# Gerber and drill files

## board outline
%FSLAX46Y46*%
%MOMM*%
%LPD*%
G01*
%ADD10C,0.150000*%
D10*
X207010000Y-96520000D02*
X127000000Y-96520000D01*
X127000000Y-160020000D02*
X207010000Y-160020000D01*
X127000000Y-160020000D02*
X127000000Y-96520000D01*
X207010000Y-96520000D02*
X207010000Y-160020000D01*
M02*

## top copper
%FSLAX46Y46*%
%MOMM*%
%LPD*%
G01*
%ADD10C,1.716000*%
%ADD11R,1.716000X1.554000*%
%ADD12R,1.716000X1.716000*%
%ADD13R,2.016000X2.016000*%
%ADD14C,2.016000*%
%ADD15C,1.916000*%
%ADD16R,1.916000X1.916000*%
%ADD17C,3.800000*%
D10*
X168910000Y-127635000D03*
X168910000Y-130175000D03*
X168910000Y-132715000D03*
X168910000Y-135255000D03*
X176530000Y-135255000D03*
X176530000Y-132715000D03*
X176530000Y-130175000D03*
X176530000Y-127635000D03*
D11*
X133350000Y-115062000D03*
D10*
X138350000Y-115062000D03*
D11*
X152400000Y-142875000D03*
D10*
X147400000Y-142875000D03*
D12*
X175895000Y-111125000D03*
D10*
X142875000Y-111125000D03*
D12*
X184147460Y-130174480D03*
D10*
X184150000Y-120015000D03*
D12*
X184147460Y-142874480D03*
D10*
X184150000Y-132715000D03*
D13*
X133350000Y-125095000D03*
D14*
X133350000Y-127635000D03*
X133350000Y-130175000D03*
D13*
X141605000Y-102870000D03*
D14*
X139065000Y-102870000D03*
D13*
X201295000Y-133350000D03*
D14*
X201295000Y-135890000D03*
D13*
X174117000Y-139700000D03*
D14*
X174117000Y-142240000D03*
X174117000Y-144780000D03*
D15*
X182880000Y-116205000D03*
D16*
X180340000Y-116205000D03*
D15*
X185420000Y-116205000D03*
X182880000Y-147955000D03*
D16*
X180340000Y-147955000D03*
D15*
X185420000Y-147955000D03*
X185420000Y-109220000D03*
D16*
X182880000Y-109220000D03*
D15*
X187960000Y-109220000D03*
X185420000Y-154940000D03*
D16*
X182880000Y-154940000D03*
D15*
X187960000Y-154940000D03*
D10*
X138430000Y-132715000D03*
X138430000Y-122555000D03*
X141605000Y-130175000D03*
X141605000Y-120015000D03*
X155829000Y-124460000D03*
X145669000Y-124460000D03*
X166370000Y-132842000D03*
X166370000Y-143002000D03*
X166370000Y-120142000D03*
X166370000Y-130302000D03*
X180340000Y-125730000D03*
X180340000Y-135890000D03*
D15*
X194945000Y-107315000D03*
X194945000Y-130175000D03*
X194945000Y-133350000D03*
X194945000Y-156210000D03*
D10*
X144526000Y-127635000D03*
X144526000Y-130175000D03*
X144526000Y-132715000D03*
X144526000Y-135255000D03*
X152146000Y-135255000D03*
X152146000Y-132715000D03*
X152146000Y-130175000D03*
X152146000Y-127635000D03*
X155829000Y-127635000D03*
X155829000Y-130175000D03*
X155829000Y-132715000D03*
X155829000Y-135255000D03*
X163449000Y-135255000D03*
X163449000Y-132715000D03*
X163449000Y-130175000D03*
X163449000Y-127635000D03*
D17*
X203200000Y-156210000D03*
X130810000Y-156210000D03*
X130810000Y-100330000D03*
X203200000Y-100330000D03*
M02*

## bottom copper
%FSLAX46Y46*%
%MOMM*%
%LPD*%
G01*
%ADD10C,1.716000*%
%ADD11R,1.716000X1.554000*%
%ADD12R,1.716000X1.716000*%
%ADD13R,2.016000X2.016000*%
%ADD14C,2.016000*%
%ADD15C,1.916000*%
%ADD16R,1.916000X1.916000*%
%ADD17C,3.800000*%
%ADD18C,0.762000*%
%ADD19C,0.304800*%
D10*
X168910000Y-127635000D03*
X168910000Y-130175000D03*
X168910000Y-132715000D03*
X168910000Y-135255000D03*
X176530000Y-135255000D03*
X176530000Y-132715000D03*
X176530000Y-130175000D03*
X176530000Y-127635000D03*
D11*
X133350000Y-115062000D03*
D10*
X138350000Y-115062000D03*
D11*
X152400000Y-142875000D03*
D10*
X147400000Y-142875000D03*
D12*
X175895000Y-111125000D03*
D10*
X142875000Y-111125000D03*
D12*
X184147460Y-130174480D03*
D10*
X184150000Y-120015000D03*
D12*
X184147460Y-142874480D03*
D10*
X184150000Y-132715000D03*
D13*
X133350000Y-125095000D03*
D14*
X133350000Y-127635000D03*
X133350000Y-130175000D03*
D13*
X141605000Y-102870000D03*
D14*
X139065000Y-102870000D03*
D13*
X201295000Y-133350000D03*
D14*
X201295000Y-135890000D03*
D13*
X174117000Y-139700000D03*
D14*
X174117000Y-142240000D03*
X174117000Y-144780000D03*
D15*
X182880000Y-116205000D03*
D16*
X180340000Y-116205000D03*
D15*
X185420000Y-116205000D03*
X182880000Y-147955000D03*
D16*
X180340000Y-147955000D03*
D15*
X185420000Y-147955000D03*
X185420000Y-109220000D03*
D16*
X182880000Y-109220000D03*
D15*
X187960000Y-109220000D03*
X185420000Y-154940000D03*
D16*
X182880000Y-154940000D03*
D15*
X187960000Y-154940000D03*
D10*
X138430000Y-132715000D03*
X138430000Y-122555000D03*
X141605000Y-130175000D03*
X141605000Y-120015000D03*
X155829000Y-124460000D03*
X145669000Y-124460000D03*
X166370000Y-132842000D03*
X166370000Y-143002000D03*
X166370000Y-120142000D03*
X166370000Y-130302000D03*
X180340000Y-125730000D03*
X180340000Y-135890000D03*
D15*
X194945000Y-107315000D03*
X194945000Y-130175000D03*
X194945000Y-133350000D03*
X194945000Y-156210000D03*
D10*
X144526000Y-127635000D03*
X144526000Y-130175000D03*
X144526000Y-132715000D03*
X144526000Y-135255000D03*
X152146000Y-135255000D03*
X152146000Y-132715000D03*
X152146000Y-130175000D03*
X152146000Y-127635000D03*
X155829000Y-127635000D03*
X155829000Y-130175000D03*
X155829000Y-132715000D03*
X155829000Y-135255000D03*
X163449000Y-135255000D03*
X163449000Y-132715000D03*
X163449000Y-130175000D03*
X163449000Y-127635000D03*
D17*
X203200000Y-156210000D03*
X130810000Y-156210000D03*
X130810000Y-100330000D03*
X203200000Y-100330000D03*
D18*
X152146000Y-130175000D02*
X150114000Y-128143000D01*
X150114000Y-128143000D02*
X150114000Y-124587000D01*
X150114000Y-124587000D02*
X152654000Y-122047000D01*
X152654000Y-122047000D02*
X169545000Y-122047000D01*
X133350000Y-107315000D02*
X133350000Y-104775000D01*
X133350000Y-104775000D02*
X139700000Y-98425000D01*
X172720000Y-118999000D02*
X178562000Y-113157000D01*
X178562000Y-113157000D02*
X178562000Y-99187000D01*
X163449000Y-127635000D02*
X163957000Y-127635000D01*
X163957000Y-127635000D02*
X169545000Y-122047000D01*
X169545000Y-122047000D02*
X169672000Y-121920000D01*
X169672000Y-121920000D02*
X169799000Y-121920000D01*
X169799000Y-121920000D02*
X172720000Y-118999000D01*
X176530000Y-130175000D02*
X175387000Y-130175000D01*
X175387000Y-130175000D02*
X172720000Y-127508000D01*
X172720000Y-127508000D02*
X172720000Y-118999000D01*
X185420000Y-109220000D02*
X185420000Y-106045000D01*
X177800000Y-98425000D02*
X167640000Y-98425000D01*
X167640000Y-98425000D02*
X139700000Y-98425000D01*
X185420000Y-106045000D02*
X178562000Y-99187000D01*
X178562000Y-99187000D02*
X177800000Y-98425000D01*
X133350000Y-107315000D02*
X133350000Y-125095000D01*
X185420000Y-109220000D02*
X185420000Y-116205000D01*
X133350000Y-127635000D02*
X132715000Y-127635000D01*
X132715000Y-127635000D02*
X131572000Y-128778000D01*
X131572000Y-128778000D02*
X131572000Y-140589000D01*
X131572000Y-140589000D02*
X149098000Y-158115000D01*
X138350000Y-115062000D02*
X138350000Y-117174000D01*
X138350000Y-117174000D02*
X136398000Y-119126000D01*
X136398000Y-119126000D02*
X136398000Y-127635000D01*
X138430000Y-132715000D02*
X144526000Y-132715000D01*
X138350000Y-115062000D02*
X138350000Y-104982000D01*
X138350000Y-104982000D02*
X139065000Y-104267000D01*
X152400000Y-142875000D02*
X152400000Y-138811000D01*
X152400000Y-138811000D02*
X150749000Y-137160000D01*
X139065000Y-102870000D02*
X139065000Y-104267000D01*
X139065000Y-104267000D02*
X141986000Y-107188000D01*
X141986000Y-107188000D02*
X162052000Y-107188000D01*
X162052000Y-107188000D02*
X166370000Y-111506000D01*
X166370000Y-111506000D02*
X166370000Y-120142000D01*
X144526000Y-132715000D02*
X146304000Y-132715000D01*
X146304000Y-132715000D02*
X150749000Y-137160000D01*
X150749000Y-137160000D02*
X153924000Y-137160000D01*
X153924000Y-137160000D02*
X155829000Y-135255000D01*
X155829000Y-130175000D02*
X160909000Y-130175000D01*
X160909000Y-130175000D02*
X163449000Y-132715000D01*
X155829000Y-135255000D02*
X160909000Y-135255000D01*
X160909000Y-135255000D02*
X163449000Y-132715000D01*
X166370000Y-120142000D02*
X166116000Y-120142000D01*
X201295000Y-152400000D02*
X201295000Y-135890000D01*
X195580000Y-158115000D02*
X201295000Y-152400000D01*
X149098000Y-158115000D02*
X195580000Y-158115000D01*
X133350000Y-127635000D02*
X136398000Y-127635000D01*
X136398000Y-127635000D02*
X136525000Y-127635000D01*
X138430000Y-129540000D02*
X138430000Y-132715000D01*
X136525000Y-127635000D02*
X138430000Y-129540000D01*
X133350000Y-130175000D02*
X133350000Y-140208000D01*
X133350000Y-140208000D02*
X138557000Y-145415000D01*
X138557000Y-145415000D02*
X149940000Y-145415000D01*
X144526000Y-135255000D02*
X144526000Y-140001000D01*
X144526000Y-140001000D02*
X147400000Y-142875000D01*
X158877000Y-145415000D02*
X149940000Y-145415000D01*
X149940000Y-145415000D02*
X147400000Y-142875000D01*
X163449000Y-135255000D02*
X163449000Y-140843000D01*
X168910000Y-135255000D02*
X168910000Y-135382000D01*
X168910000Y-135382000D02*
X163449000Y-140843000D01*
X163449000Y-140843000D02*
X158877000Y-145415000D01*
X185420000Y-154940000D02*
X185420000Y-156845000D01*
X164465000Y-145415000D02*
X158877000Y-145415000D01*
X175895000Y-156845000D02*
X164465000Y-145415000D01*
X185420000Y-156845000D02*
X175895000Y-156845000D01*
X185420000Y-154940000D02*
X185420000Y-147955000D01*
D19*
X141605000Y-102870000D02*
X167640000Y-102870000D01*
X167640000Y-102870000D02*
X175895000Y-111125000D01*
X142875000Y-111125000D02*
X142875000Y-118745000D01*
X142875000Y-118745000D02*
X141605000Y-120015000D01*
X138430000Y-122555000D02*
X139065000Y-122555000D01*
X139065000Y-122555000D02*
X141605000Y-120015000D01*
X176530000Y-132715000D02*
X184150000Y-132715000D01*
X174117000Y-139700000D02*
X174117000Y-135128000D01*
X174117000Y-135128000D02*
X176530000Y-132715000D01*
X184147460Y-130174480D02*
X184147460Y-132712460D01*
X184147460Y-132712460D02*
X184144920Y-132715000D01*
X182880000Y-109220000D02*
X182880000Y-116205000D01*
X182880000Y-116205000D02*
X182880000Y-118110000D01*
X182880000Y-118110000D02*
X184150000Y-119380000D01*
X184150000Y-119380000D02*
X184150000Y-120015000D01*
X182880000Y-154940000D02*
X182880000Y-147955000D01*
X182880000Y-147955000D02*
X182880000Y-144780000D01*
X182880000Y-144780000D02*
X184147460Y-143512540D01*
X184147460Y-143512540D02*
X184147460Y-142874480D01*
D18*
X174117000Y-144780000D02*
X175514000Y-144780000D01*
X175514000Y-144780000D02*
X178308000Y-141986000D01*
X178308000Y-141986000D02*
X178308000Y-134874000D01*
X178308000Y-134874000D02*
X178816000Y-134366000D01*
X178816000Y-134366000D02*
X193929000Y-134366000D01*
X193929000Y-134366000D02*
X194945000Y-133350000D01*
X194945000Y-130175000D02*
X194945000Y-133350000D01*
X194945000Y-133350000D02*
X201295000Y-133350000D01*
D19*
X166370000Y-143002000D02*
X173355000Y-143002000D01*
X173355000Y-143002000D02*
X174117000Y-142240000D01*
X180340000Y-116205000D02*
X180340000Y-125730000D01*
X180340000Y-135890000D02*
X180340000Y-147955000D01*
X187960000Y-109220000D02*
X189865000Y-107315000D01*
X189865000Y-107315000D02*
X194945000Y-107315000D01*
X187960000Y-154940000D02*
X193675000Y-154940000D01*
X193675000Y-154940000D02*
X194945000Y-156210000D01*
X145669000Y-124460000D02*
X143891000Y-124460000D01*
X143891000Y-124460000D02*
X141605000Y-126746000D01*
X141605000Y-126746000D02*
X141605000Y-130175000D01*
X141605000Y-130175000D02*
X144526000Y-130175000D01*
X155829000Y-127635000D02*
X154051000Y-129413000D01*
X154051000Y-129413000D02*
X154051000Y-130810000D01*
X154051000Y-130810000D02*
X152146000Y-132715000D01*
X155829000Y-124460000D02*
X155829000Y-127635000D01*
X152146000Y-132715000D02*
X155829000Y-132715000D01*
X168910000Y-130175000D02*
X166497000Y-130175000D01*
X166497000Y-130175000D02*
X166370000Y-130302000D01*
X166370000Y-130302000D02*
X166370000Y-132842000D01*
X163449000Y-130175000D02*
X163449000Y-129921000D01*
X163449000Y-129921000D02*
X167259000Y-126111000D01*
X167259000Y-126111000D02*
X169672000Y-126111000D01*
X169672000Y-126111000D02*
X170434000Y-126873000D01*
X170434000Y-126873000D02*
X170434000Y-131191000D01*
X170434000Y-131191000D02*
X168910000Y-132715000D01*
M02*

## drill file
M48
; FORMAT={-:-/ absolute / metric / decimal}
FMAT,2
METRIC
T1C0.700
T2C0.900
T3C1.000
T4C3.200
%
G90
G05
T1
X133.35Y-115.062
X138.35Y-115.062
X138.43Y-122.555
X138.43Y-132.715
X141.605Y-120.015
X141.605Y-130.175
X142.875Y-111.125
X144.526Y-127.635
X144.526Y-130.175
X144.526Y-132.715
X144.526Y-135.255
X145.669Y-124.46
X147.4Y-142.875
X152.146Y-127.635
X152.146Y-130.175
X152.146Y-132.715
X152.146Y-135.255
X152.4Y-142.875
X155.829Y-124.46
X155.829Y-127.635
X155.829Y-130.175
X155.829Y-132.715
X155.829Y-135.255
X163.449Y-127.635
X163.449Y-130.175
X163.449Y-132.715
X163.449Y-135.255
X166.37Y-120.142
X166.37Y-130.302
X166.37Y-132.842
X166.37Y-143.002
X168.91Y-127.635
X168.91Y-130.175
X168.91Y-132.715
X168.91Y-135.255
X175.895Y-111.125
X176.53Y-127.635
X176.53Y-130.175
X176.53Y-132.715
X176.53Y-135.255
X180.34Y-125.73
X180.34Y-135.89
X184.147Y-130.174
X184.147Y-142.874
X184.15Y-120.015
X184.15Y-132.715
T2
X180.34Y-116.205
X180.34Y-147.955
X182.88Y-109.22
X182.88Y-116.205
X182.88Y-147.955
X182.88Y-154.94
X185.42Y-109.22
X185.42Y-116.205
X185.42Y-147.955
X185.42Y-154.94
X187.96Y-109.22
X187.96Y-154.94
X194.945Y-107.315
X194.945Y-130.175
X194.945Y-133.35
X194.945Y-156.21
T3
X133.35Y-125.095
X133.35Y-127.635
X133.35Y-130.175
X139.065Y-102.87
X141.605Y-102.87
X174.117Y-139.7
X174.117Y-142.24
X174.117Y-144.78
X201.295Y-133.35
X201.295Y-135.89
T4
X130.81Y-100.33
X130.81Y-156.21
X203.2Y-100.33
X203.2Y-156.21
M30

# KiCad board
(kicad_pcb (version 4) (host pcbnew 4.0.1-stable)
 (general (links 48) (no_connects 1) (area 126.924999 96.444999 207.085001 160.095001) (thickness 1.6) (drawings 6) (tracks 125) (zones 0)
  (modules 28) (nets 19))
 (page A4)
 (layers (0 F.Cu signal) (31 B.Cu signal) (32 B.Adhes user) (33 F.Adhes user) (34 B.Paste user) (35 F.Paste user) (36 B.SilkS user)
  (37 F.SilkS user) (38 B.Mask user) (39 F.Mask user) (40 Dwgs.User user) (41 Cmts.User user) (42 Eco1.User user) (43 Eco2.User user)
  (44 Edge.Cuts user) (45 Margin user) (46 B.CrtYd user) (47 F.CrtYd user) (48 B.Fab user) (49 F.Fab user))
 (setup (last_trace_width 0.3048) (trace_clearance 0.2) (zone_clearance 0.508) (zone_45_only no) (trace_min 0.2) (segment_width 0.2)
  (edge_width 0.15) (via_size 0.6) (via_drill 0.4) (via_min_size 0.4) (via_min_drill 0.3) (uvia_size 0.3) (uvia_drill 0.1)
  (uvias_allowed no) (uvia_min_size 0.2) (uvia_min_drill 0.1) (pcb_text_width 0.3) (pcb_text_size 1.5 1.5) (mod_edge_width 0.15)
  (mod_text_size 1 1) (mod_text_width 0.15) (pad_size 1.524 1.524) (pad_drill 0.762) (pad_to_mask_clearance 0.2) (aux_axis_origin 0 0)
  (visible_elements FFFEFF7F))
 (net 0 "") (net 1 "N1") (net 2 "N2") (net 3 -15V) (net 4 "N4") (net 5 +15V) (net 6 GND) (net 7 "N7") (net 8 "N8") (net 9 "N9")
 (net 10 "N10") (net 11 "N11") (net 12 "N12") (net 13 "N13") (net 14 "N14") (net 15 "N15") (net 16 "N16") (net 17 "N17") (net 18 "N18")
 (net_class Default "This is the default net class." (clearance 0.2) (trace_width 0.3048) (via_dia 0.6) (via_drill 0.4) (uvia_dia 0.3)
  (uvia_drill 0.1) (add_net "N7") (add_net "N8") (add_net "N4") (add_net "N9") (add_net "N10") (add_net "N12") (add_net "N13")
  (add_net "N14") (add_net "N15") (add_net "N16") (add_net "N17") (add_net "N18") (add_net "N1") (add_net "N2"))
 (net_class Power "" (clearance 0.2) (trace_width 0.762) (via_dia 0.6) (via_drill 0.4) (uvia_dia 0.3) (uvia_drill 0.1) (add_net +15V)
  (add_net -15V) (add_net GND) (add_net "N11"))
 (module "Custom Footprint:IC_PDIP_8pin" (layer F.Cu) (at 172.72 131.445 270)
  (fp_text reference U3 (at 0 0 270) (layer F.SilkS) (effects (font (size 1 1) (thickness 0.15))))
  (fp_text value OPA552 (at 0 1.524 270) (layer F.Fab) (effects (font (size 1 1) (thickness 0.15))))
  (pad 1 thru_hole circle (at -3.81 3.81 270) (size 1.716 1.716) (drill 0.7) (layers *.Cu *.Mask F.SilkS))
  (pad 2 thru_hole circle (at -1.27 3.81 270) (size 1.716 1.716) (drill 0.7) (layers *.Cu *.Mask F.SilkS) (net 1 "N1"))
  (pad 3 thru_hole circle (at 1.27 3.81 270) (size 1.716 1.716) (drill 0.7) (layers *.Cu *.Mask F.SilkS) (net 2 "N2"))
  (pad 4 thru_hole circle (at 3.81 3.81 270) (size 1.716 1.716) (drill 0.7) (layers *.Cu *.Mask F.SilkS) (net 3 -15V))
  (pad 5 thru_hole circle (at 3.81 -3.81 270) (size 1.716 1.716) (drill 0.7) (layers *.Cu *.Mask F.SilkS))
  (pad 6 thru_hole circle (at 1.27 -3.81 270) (size 1.716 1.716) (drill 0.7) (layers *.Cu *.Mask F.SilkS) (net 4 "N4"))
  (pad 7 thru_hole circle (at -1.27 -3.81 270) (size 1.716 1.716) (drill 0.7) (layers *.Cu *.Mask F.SilkS) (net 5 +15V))
  (pad 8 thru_hole circle (at -3.81 -3.81 270) (size 1.716 1.716) (drill 0.7) (layers *.Cu *.Mask F.SilkS)))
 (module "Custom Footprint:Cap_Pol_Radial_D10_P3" (layer F.Cu) (at 133.35 115.062)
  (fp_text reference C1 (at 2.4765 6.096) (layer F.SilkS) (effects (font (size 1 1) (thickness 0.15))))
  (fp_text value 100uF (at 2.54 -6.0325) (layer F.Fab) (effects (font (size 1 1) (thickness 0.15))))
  (pad 1 thru_hole rect (at 0 0) (size 1.716 1.554) (drill 0.7) (layers *.Cu *.Mask F.SilkS) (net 5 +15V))
  (pad 2 thru_hole circle (at 5 0) (size 1.716 1.716) (drill 0.7) (layers *.Cu *.Mask F.SilkS) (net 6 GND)))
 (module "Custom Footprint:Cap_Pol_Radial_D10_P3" (layer F.Cu) (at 152.4 142.875 180)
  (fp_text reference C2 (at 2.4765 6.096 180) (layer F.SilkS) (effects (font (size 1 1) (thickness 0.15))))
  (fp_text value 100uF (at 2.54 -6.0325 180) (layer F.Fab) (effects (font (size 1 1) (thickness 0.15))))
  (pad 1 thru_hole rect (at 0 0 180) (size 1.716 1.554) (drill 0.7) (layers *.Cu *.Mask F.SilkS) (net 6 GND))
  (pad 2 thru_hole circle (at 5 0 180) (size 1.716 1.716) (drill 0.7) (layers *.Cu *.Mask F.SilkS) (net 3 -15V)))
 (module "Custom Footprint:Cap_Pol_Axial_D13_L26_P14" (layer F.Cu) (at 175.895 111.125 180)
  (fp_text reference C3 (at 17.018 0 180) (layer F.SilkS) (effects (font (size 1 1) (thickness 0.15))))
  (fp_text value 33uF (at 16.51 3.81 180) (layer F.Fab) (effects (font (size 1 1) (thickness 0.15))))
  (pad 1 thru_hole rect (at 0 0 180) (size 1.716 1.716) (drill 0.7) (layers *.Cu *.Mask F.SilkS) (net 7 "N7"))
  (pad 2 thru_hole circle (at 33.02 0 180) (size 1.716 1.716) (drill 0.7) (layers *.Cu *.Mask F.SilkS) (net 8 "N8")))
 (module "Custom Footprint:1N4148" (layer F.Cu) (at 184.15 130.175 90)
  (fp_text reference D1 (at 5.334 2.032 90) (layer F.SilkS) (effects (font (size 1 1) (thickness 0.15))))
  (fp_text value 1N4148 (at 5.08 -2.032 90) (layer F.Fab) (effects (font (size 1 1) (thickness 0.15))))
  (pad 1 thru_hole rect (at 0.00052 -0.00254 270) (size 1.716 1.716) (drill 0.7) (layers *.Cu *.Mask F.SilkS) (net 4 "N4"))
  (pad 2 thru_hole circle (at 10.16 0 90) (size 1.716 1.716) (drill 0.7) (layers *.Cu *.Mask F.SilkS) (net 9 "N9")))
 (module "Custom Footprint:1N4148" (layer F.Cu) (at 184.15 142.875 90)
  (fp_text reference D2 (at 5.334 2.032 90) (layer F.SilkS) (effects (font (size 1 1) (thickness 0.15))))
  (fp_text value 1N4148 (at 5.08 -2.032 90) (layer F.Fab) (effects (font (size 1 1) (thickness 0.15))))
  (pad 1 thru_hole rect (at 0.00052 -0.00254 270) (size 1.716 1.716) (drill 0.7) (layers *.Cu *.Mask F.SilkS) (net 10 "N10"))
  (pad 2 thru_hole circle (at 10.16 0 90) (size 1.716 1.716) (drill 0.7) (layers *.Cu *.Mask F.SilkS) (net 4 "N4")))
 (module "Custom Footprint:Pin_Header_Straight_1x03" (layer F.Cu) (at 133.35 125.095)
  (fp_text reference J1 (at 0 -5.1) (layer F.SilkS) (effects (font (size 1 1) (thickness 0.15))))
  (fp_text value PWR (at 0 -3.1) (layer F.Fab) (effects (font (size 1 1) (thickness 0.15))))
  (pad 1 thru_hole rect (at 0 0) (size 2.016 2.016) (drill 1) (layers *.Cu *.Mask F.SilkS) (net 5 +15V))
  (pad 2 thru_hole circle (at 0 2.54) (size 2.016 2.016) (drill 1) (layers *.Cu *.Mask F.SilkS) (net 6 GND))
  (pad 3 thru_hole circle (at 0 5.08) (size 2.016 2.016) (drill 1) (layers *.Cu *.Mask F.SilkS) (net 3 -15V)))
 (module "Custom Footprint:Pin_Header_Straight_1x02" (layer F.Cu) (at 141.605 102.87 270)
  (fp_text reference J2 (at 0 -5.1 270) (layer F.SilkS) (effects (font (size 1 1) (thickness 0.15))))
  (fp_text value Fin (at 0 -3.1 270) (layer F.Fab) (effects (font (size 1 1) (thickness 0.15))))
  (pad 1 thru_hole rect (at 0 0 270) (size 2.016 2.016) (drill 1) (layers *.Cu *.Mask F.SilkS) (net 7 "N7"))
  (pad 2 thru_hole circle (at 0 2.54 270) (size 2.016 2.016) (drill 1) (layers *.Cu *.Mask F.SilkS) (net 6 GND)))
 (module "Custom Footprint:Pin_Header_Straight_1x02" (layer F.Cu) (at 201.295 133.35)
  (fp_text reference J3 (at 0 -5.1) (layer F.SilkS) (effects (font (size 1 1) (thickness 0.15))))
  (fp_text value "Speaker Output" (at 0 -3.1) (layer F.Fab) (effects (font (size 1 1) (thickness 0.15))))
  (pad 1 thru_hole rect (at 0 0) (size 2.016 2.016) (drill 1) (layers *.Cu *.Mask F.SilkS) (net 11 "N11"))
  (pad 2 thru_hole circle (at 0 2.54) (size 2.016 2.016) (drill 1) (layers *.Cu *.Mask F.SilkS) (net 6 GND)))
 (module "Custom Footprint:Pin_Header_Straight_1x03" (layer F.Cu) (at 174.117 139.7)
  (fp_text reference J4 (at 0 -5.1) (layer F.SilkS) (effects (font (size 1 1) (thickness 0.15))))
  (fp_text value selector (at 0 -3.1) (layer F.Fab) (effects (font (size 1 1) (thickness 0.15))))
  (pad 1 thru_hole rect (at 0 0) (size 2.016 2.016) (drill 1) (layers *.Cu *.Mask F.SilkS) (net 4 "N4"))
  (pad 2 thru_hole circle (at 0 2.54) (size 2.016 2.016) (drill 1) (layers *.Cu *.Mask F.SilkS) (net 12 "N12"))
  (pad 3 thru_hole circle (at 0 5.08) (size 2.016 2.016) (drill 1) (layers *.Cu *.Mask F.SilkS) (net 11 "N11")))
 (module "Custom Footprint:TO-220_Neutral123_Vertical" (layer F.Cu) (at 182.88 116.205)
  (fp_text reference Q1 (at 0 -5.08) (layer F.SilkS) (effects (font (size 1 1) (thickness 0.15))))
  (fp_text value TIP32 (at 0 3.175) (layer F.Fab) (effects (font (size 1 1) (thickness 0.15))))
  (pad 2 thru_hole circle (at 0 0 90) (size 1.916 1.916) (drill 0.9) (layers *.Cu *.Mask F.SilkS) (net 9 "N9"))
  (pad 1 thru_hole rect (at -2.54 0 90) (size 1.916 1.916) (drill 0.9) (layers *.Cu *.Mask F.SilkS) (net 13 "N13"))
  (pad 3 thru_hole circle (at 2.54 0 90) (size 1.916 1.916) (drill 0.9) (layers *.Cu *.Mask F.SilkS) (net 5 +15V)))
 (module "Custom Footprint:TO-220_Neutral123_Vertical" (layer F.Cu) (at 182.88 147.955)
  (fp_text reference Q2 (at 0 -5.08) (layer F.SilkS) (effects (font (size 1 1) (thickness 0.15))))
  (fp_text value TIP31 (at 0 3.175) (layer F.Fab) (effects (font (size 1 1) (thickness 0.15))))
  (pad 2 thru_hole circle (at 0 0 90) (size 1.916 1.916) (drill 0.9) (layers *.Cu *.Mask F.SilkS) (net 10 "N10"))
  (pad 1 thru_hole rect (at -2.54 0 90) (size 1.916 1.916) (drill 0.9) (layers *.Cu *.Mask F.SilkS) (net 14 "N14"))
  (pad 3 thru_hole circle (at 2.54 0 90) (size 1.916 1.916) (drill 0.9) (layers *.Cu *.Mask F.SilkS) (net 3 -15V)))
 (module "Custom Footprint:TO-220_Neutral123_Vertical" (layer F.Cu) (at 185.42 109.22)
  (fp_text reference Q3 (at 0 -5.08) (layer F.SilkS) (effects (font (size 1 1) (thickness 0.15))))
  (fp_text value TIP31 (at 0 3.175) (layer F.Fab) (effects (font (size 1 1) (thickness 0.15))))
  (pad 2 thru_hole circle (at 0 0 90) (size 1.916 1.916) (drill 0.9) (layers *.Cu *.Mask F.SilkS) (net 5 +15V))
  (pad 1 thru_hole rect (at -2.54 0 90) (size 1.916 1.916) (drill 0.9) (layers *.Cu *.Mask F.SilkS) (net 9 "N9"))
  (pad 3 thru_hole circle (at 2.54 0 90) (size 1.916 1.916) (drill 0.9) (layers *.Cu *.Mask F.SilkS) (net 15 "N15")))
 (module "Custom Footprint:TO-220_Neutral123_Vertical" (layer F.Cu) (at 185.42 154.94)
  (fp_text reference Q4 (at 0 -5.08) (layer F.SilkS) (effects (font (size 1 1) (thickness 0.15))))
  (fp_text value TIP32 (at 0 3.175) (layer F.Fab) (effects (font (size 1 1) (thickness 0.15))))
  (pad 2 thru_hole circle (at 0 0 90) (size 1.916 1.916) (drill 0.9) (layers *.Cu *.Mask F.SilkS) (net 3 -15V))
  (pad 1 thru_hole rect (at -2.54 0 90) (size 1.916 1.916) (drill 0.9) (layers *.Cu *.Mask F.SilkS) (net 10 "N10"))
  (pad 3 thru_hole circle (at 2.54 0 90) (size 1.916 1.916) (drill 0.9) (layers *.Cu *.Mask F.SilkS) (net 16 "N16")))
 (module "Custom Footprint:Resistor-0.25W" (layer F.Cu) (at 138.43 132.715 90)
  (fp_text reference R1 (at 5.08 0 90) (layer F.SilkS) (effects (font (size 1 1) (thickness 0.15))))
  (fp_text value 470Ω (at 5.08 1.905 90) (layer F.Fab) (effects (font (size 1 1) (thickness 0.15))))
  (pad 1 thru_hole circle (at 0 0 90) (size 1.716 1.716) (drill 0.7) (layers *.Cu *.Mask F.SilkS) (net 6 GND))
  (pad 2 thru_hole circle (at 10.16 0 90) (size 1.716 1.716) (drill 0.7) (layers *.Cu *.Mask F.SilkS) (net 8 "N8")))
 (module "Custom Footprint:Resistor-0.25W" (layer F.Cu) (at 141.605 130.175 90)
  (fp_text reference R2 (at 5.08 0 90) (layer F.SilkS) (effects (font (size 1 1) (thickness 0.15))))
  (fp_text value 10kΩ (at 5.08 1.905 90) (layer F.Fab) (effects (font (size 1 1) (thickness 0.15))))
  (pad 1 thru_hole circle (at 0 0 90) (size 1.716 1.716) (drill 0.7) (layers *.Cu *.Mask F.SilkS) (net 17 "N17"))
  (pad 2 thru_hole circle (at 10.16 0 90) (size 1.716 1.716) (drill 0.7) (layers *.Cu *.Mask F.SilkS) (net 8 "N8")))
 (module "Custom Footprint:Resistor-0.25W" (layer F.Cu) (at 155.829 124.46 180)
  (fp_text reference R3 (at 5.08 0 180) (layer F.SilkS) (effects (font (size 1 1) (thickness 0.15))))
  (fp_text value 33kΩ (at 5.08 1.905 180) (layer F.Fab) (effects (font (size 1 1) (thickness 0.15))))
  (pad 1 thru_hole circle (at 0 0 180) (size 1.716 1.716) (drill 0.7) (layers *.Cu *.Mask F.SilkS) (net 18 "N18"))
  (pad 2 thru_hole circle (at 10.16 0 180) (size 1.716 1.716) (drill 0.7) (layers *.Cu *.Mask F.SilkS) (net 17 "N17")))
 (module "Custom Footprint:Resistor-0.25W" (layer F.Cu) (at 166.37 132.842 270)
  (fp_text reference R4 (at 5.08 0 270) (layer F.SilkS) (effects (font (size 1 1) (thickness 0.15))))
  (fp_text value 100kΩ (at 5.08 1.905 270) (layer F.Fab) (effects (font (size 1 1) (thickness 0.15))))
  (pad 1 thru_hole circle (at 0 0 270) (size 1.716 1.716) (drill 0.7) (layers *.Cu *.Mask F.SilkS) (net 1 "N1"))
  (pad 2 thru_hole circle (at 10.16 0 270) (size 1.716 1.716) (drill 0.7) (layers *.Cu *.Mask F.SilkS) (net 12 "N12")))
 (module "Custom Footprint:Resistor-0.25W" (layer F.Cu) (at 166.37 120.142 270)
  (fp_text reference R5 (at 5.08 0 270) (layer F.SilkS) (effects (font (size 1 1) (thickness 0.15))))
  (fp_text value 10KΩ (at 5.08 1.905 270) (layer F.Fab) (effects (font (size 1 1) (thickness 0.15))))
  (pad 1 thru_hole circle (at 0 0 270) (size 1.716 1.716) (drill 0.7) (layers *.Cu *.Mask F.SilkS) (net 6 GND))
  (pad 2 thru_hole circle (at 10.16 0 270) (size 1.716 1.716) (drill 0.7) (layers *.Cu *.Mask F.SilkS) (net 1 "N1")))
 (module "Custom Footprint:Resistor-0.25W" (layer F.Cu) (at 180.34 125.73 270)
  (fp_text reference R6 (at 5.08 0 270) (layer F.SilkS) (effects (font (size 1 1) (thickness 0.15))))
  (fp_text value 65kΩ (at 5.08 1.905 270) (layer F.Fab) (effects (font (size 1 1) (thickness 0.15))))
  (pad 1 thru_hole circle (at 0 0 270) (size 1.716 1.716) (drill 0.7) (layers *.Cu *.Mask F.SilkS) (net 13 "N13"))
  (pad 2 thru_hole circle (at 10.16 0 270) (size 1.716 1.716) (drill 0.7) (layers *.Cu *.Mask F.SilkS) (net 14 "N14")))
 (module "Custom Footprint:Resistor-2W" (layer F.Cu) (at 194.945 107.315 270)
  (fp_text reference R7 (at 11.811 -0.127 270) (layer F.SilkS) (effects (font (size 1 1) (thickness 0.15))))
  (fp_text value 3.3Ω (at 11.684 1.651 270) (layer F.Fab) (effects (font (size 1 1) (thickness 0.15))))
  (pad 1 thru_hole circle (at 0 0 270) (size 1.916 1.916) (drill 0.9) (layers *.Cu *.SilkS *.Mask) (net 15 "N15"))
  (pad 2 thru_hole circle (at 22.86 0 270) (size 1.916 1.916) (drill 0.9) (layers *.Cu *.SilkS *.Mask) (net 11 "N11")))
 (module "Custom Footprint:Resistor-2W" (layer F.Cu) (at 194.945 133.35 270)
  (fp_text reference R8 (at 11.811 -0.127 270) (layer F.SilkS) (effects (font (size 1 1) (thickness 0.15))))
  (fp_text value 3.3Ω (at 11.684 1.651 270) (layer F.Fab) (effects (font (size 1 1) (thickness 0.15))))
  (pad 1 thru_hole circle (at 0 0 270) (size 1.916 1.916) (drill 0.9) (layers *.Cu *.SilkS *.Mask) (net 11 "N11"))
  (pad 2 thru_hole circle (at 22.86 0 270) (size 1.916 1.916) (drill 0.9) (layers *.Cu *.SilkS *.Mask) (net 16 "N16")))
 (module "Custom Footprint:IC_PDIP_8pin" (layer F.Cu) (at 148.336 131.445 270)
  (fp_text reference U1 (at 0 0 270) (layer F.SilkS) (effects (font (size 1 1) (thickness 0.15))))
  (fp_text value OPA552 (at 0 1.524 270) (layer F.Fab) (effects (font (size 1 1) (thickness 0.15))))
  (pad 1 thru_hole circle (at -3.81 3.81 270) (size 1.716 1.716) (drill 0.7) (layers *.Cu *.Mask F.SilkS))
  (pad 2 thru_hole circle (at -1.27 3.81 270) (size 1.716 1.716) (drill 0.7) (layers *.Cu *.Mask F.SilkS) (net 17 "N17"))
  (pad 3 thru_hole circle (at 1.27 3.81 270) (size 1.716 1.716) (drill 0.7) (layers *.Cu *.Mask F.SilkS) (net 6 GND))
  (pad 4 thru_hole circle (at 3.81 3.81 270) (size 1.716 1.716) (drill 0.7) (layers *.Cu *.Mask F.SilkS) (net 3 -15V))
  (pad 5 thru_hole circle (at 3.81 -3.81 270) (size 1.716 1.716) (drill 0.7) (layers *.Cu *.Mask F.SilkS))
  (pad 6 thru_hole circle (at 1.27 -3.81 270) (size 1.716 1.716) (drill 0.7) (layers *.Cu *.Mask F.SilkS) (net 18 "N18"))
  (pad 7 thru_hole circle (at -1.27 -3.81 270) (size 1.716 1.716) (drill 0.7) (layers *.Cu *.Mask F.SilkS) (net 5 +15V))
  (pad 8 thru_hole circle (at -3.81 -3.81 270) (size 1.716 1.716) (drill 0.7) (layers *.Cu *.Mask F.SilkS)))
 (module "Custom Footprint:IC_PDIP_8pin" (layer F.Cu) (at 159.639 131.445 270)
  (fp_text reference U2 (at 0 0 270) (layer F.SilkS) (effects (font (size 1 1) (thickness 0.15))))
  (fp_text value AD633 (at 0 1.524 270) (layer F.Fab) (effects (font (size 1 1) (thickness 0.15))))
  (pad 1 thru_hole circle (at -3.81 3.81 270) (size 1.716 1.716) (drill 0.7) (layers *.Cu *.Mask F.SilkS) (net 18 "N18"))
  (pad 2 thru_hole circle (at -1.27 3.81 270) (size 1.716 1.716) (drill 0.7) (layers *.Cu *.Mask F.SilkS) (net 6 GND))
  (pad 3 thru_hole circle (at 1.27 3.81 270) (size 1.716 1.716) (drill 0.7) (layers *.Cu *.Mask F.SilkS) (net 18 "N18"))
  (pad 4 thru_hole circle (at 3.81 3.81 270) (size 1.716 1.716) (drill 0.7) (layers *.Cu *.Mask F.SilkS) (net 6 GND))
  (pad 5 thru_hole circle (at 3.81 -3.81 270) (size 1.716 1.716) (drill 0.7) (layers *.Cu *.Mask F.SilkS) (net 3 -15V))
  (pad 6 thru_hole circle (at 1.27 -3.81 270) (size 1.716 1.716) (drill 0.7) (layers *.Cu *.Mask F.SilkS) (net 6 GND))
  (pad 7 thru_hole circle (at -1.27 -3.81 270) (size 1.716 1.716) (drill 0.7) (layers *.Cu *.Mask F.SilkS) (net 2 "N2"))
  (pad 8 thru_hole circle (at -3.81 -3.81 270) (size 1.716 1.716) (drill 0.7) (layers *.Cu *.Mask F.SilkS) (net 5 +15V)))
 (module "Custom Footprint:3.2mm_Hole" (layer F.Cu) (at 203.2 156.21)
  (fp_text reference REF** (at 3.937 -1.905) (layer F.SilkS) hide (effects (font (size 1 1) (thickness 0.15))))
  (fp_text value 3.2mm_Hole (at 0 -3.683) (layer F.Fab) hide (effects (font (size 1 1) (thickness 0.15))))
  (pad 1 thru_hole circle (at 0 0) (size 3.8 3.8) (drill 3.2) (layers *.Cu *.Mask F.SilkS)))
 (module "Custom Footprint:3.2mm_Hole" (layer F.Cu) (at 130.81 156.21)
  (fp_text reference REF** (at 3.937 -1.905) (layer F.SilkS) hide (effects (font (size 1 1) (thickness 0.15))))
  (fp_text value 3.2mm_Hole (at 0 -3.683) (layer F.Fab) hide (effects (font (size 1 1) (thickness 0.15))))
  (pad 1 thru_hole circle (at 0 0) (size 3.8 3.8) (drill 3.2) (layers *.Cu *.Mask F.SilkS)))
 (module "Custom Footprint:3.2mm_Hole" (layer F.Cu) (at 130.81 100.33)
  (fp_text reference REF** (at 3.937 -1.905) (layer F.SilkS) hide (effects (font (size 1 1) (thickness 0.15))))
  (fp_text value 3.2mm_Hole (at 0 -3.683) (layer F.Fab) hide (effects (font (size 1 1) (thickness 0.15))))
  (pad 1 thru_hole circle (at 0 0) (size 3.8 3.8) (drill 3.2) (layers *.Cu *.Mask F.SilkS)))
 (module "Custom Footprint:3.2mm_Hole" (layer F.Cu) (at 203.2 100.33)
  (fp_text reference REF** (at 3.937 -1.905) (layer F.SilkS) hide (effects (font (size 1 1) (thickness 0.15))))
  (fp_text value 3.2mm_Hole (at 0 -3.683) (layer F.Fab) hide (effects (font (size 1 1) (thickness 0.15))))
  (pad 1 thru_hole circle (at 0 0) (size 3.8 3.8) (drill 3.2) (layers *.Cu *.Mask F.SilkS)))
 (gr_line (start 207.01 96.52) (end 127 96.52) (angle 90) (layer Edge.Cuts) (width 0.15))
 (gr_line (start 127 160.02) (end 207.01 160.02) (angle 90) (layer Edge.Cuts) (width 0.15))
 (gr_line (start 127 160.02) (end 127 96.52) (angle 90) (layer Edge.Cuts) (width 0.15))
 (gr_line (start 207.01 96.52) (end 207.01 160.02) (angle 90) (layer Edge.Cuts) (width 0.15))
 (segment (start 152.146 130.175) (end 150.114 128.143) (width 0.762) (layer B.Cu) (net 5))
 (segment (start 150.114 128.143) (end 150.114 124.587) (width 0.762) (layer B.Cu) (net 5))
 (segment (start 150.114 124.587) (end 152.654 122.047) (width 0.762) (layer B.Cu) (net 5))
 (segment (start 152.654 122.047) (end 169.545 122.047) (width 0.762) (layer B.Cu) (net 5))
 (segment (start 133.35 107.315) (end 133.35 104.775) (width 0.762) (layer B.Cu) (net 5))
 (segment (start 133.35 104.775) (end 139.7 98.425) (width 0.762) (layer B.Cu) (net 5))
 (segment (start 172.72 118.999) (end 178.562 113.157) (width 0.762) (layer B.Cu) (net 5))
 (segment (start 178.562 113.157) (end 178.562 99.187) (width 0.762) (layer B.Cu) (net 5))
 (segment (start 163.449 127.635) (end 163.957 127.635) (width 0.762) (layer B.Cu) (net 5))
 (segment (start 163.957 127.635) (end 169.545 122.047) (width 0.762) (layer B.Cu) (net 5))
 (segment (start 169.545 122.047) (end 169.672 121.92) (width 0.762) (layer B.Cu) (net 5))
 (segment (start 169.672 121.92) (end 169.799 121.92) (width 0.762) (layer B.Cu) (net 5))
 (segment (start 169.799 121.92) (end 172.72 118.999) (width 0.762) (layer B.Cu) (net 5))
 (segment (start 176.53 130.175) (end 175.387 130.175) (width 0.762) (layer B.Cu) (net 5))
 (segment (start 175.387 130.175) (end 172.72 127.508) (width 0.762) (layer B.Cu) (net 5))
 (segment (start 172.72 127.508) (end 172.72 118.999) (width 0.762) (layer B.Cu) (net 5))
 (segment (start 185.42 109.22) (end 185.42 106.045) (width 0.762) (layer B.Cu) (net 5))
 (segment (start 177.8 98.425) (end 167.64 98.425) (width 0.762) (layer B.Cu) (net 5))
 (segment (start 167.64 98.425) (end 139.7 98.425) (width 0.762) (layer B.Cu) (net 5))
 (segment (start 185.42 106.045) (end 178.562 99.187) (width 0.762) (layer B.Cu) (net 5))
 (segment (start 178.562 99.187) (end 177.8 98.425) (width 0.762) (layer B.Cu) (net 5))
 (segment (start 133.35 107.315) (end 133.35 125.095) (width 0.762) (layer B.Cu) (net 5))
 (segment (start 185.42 109.22) (end 185.42 116.205) (width 0.762) (layer B.Cu) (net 5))
 (segment (start 133.35 127.635) (end 132.715 127.635) (width 0.762) (layer B.Cu) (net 6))
 (segment (start 132.715 127.635) (end 131.572 128.778) (width 0.762) (layer B.Cu) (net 6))
 (segment (start 131.572 128.778) (end 131.572 140.589) (width 0.762) (layer B.Cu) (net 6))
 (segment (start 131.572 140.589) (end 149.098 158.115) (width 0.762) (layer B.Cu) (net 6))
 (segment (start 138.35 115.062) (end 138.35 117.174) (width 0.762) (layer B.Cu) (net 6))
 (segment (start 138.35 117.174) (end 136.398 119.126) (width 0.762) (layer B.Cu) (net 6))
 (segment (start 136.398 119.126) (end 136.398 127.635) (width 0.762) (layer B.Cu) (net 6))
 (segment (start 138.43 132.715) (end 144.526 132.715) (width 0.762) (layer B.Cu) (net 6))
 (segment (start 138.35 115.062) (end 138.35 104.982) (width 0.762) (layer B.Cu) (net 6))
 (segment (start 138.35 104.982) (end 139.065 104.267) (width 0.762) (layer B.Cu) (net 6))
 (segment (start 152.4 142.875) (end 152.4 138.811) (width 0.762) (layer B.Cu) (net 6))
 (segment (start 152.4 138.811) (end 150.749 137.16) (width 0.762) (layer B.Cu) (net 6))
 (segment (start 139.065 102.87) (end 139.065 104.267) (width 0.762) (layer B.Cu) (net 6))
 (segment (start 139.065 104.267) (end 141.986 107.188) (width 0.762) (layer B.Cu) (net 6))
 (segment (start 141.986 107.188) (end 162.052 107.188) (width 0.762) (layer B.Cu) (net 6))
 (segment (start 162.052 107.188) (end 166.37 111.506) (width 0.762) (layer B.Cu) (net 6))
 (segment (start 166.37 111.506) (end 166.37 120.142) (width 0.762) (layer B.Cu) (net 6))
 (segment (start 144.526 132.715) (end 146.304 132.715) (width 0.762) (layer B.Cu) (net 6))
 (segment (start 146.304 132.715) (end 150.749 137.16) (width 0.762) (layer B.Cu) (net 6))
 (segment (start 150.749 137.16) (end 153.924 137.16) (width 0.762) (layer B.Cu) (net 6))
 (segment (start 153.924 137.16) (end 155.829 135.255) (width 0.762) (layer B.Cu) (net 6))
 (segment (start 155.829 130.175) (end 160.909 130.175) (width 0.762) (layer B.Cu) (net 6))
 (segment (start 160.909 130.175) (end 163.449 132.715) (width 0.762) (layer B.Cu) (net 6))
 (segment (start 155.829 135.255) (end 160.909 135.255) (width 0.762) (layer B.Cu) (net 6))
 (segment (start 160.909 135.255) (end 163.449 132.715) (width 0.762) (layer B.Cu) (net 6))
 (segment (start 166.37 120.142) (end 166.116 120.142) (width 0.762) (layer B.Cu) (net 6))
 (segment (start 201.295 152.4) (end 201.295 135.89) (width 0.762) (layer B.Cu) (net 6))
 (segment (start 195.58 158.115) (end 201.295 152.4) (width 0.762) (layer B.Cu) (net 6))
 (segment (start 149.098 158.115) (end 195.58 158.115) (width 0.762) (layer B.Cu) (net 6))
 (segment (start 133.35 127.635) (end 136.398 127.635) (width 0.762) (layer B.Cu) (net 6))
 (segment (start 136.398 127.635) (end 136.525 127.635) (width 0.762) (layer B.Cu) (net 6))
 (segment (start 138.43 129.54) (end 138.43 132.715) (width 0.762) (layer B.Cu) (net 6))
 (segment (start 136.525 127.635) (end 138.43 129.54) (width 0.762) (layer B.Cu) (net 6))
 (segment (start 133.35 130.175) (end 133.35 140.208) (width 0.762) (layer B.Cu) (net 3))
 (segment (start 133.35 140.208) (end 138.557 145.415) (width 0.762) (layer B.Cu) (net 3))
 (segment (start 138.557 145.415) (end 149.94 145.415) (width 0.762) (layer B.Cu) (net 3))
 (segment (start 144.526 135.255) (end 144.526 140.001) (width 0.762) (layer B.Cu) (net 3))
 (segment (start 144.526 140.001) (end 147.4 142.875) (width 0.762) (layer B.Cu) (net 3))
 (segment (start 158.877 145.415) (end 149.94 145.415) (width 0.762) (layer B.Cu) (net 3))
 (segment (start 149.94 145.415) (end 147.4 142.875) (width 0.762) (layer B.Cu) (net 3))
 (segment (start 163.449 135.255) (end 163.449 140.843) (width 0.762) (layer B.Cu) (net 3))
 (segment (start 168.91 135.255) (end 168.91 135.382) (width 0.762) (layer B.Cu) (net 3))
 (segment (start 168.91 135.382) (end 163.449 140.843) (width 0.762) (layer B.Cu) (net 3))
 (segment (start 163.449 140.843) (end 158.877 145.415) (width 0.762) (layer B.Cu) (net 3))
 (segment (start 185.42 154.94) (end 185.42 156.845) (width 0.762) (layer B.Cu) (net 3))
 (segment (start 164.465 145.415) (end 158.877 145.415) (width 0.762) (layer B.Cu) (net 3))
 (segment (start 175.895 156.845) (end 164.465 145.415) (width 0.762) (layer B.Cu) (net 3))
 (segment (start 185.42 156.845) (end 175.895 156.845) (width 0.762) (layer B.Cu) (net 3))
 (segment (start 185.42 154.94) (end 185.42 147.955) (width 0.762) (layer B.Cu) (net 3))
 (segment (start 141.605 102.87) (end 167.64 102.87) (width 0.3048) (layer B.Cu) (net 7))
 (segment (start 167.64 102.87) (end 175.895 111.125) (width 0.3048) (layer B.Cu) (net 7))
 (segment (start 142.875 111.125) (end 142.875 118.745) (width 0.3048) (layer B.Cu) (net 8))
 (segment (start 142.875 118.745) (end 141.605 120.015) (width 0.3048) (layer B.Cu) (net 8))
 (segment (start 138.43 122.555) (end 139.065 122.555) (width 0.3048) (layer B.Cu) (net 8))
 (segment (start 139.065 122.555) (end 141.605 120.015) (width 0.3048) (layer B.Cu) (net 8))
 (segment (start 176.53 132.715) (end 184.15 132.715) (width 0.3048) (layer B.Cu) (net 4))
 (segment (start 174.117 139.7) (end 174.117 135.128) (width 0.3048) (layer B.Cu) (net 4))
 (segment (start 174.117 135.128) (end 176.53 132.715) (width 0.3048) (layer B.Cu) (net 4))
 (segment (start 184.14746 130.17448) (end 184.14746 132.71246) (width 0.3048) (layer B.Cu) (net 4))
 (segment (start 184.14746 132.71246) (end 184.14492 132.715) (width 0.3048) (layer B.Cu) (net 4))
 (segment (start 182.88 109.22) (end 182.88 116.205) (width 0.3048) (layer B.Cu) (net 9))
 (segment (start 182.88 116.205) (end 182.88 118.11) (width 0.3048) (layer B.Cu) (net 9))
 (segment (start 182.88 118.11) (end 184.15 119.38) (width 0.3048) (layer B.Cu) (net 9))
 (segment (start 184.15 119.38) (end 184.15 120.015) (width 0.3048) (layer B.Cu) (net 9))
 (segment (start 182.88 154.94) (end 182.88 147.955) (width 0.3048) (layer B.Cu) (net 10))
 (segment (start 182.88 147.955) (end 182.88 144.78) (width 0.3048) (layer B.Cu) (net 10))
 (segment (start 182.88 144.78) (end 184.14746 143.51254) (width 0.3048) (layer B.Cu) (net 10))
 (segment (start 184.14746 143.51254) (end 184.14746 142.87448) (width 0.3048) (layer B.Cu) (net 10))
 (segment (start 174.117 144.78) (end 175.514 144.78) (width 0.762) (layer B.Cu) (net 11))
 (segment (start 175.514 144.78) (end 178.308 141.986) (width 0.762) (layer B.Cu) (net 11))
 (segment (start 178.308 141.986) (end 178.308 134.874) (width 0.762) (layer B.Cu) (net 11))
 (segment (start 178.308 134.874) (end 178.816 134.366) (width 0.762) (layer B.Cu) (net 11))
 (segment (start 178.816 134.366) (end 193.929 134.366) (width 0.762) (layer B.Cu) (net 11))
 (segment (start 193.929 134.366) (end 194.945 133.35) (width 0.762) (layer B.Cu) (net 11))
 (segment (start 194.945 130.175) (end 194.945 133.35) (width 0.762) (layer B.Cu) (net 11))
 (segment (start 194.945 133.35) (end 201.295 133.35) (width 0.762) (layer B.Cu) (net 11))
 (segment (start 166.37 143.002) (end 173.355 143.002) (width 0.3048) (layer B.Cu) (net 12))
 (segment (start 173.355 143.002) (end 174.117 142.24) (width 0.3048) (layer B.Cu) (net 12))
 (segment (start 180.34 116.205) (end 180.34 125.73) (width 0.3048) (layer B.Cu) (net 13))
 (segment (start 180.34 135.89) (end 180.34 147.955) (width 0.3048) (layer B.Cu) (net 14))
 (segment (start 187.96 109.22) (end 189.865 107.315) (width 0.3048) (layer B.Cu) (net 15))
 (segment (start 189.865 107.315) (end 194.945 107.315) (width 0.3048) (layer B.Cu) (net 15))
 (segment (start 187.96 154.94) (end 193.675 154.94) (width 0.3048) (layer B.Cu) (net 16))
 (segment (start 193.675 154.94) (end 194.945 156.21) (width 0.3048) (layer B.Cu) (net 16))
 (segment (start 145.669 124.46) (end 143.891 124.46) (width 0.3048) (layer B.Cu) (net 17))
 (segment (start 143.891 124.46) (end 141.605 126.746) (width 0.3048) (layer B.Cu) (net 17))
 (segment (start 141.605 126.746) (end 141.605 130.175) (width 0.3048) (layer B.Cu) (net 17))
 (segment (start 141.605 130.175) (end 144.526 130.175) (width 0.3048) (layer B.Cu) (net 17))
 (segment (start 155.829 127.635) (end 154.051 129.413) (width 0.3048) (layer B.Cu) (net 18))
 (segment (start 154.051 129.413) (end 154.051 130.81) (width 0.3048) (layer B.Cu) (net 18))
 (segment (start 154.051 130.81) (end 152.146 132.715) (width 0.3048) (layer B.Cu) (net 18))
 (segment (start 155.829 124.46) (end 155.829 127.635) (width 0.3048) (layer B.Cu) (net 18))
 (segment (start 152.146 132.715) (end 155.829 132.715) (width 0.3048) (layer B.Cu) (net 18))
 (segment (start 168.91 130.175) (end 166.497 130.175) (width 0.3048) (layer B.Cu) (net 1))
 (segment (start 166.497 130.175) (end 166.37 130.302) (width 0.3048) (layer B.Cu) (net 1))
 (segment (start 166.37 130.302) (end 166.37 132.842) (width 0.3048) (layer B.Cu) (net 1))
 (segment (start 163.449 130.175) (end 163.449 129.921) (width 0.3048) (layer B.Cu) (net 2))
 (segment (start 163.449 129.921) (end 167.259 126.111) (width 0.3048) (layer B.Cu) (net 2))
 (segment (start 167.259 126.111) (end 169.672 126.111) (width 0.3048) (layer B.Cu) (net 2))
 (segment (start 169.672 126.111) (end 170.434 126.873) (width 0.3048) (layer B.Cu) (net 2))
 (segment (start 170.434 126.873) (end 170.434 131.191) (width 0.3048) (layer B.Cu) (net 2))
 (segment (start 170.434 131.191) (end 168.91 132.715) (width 0.3048) (layer B.Cu) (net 2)))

